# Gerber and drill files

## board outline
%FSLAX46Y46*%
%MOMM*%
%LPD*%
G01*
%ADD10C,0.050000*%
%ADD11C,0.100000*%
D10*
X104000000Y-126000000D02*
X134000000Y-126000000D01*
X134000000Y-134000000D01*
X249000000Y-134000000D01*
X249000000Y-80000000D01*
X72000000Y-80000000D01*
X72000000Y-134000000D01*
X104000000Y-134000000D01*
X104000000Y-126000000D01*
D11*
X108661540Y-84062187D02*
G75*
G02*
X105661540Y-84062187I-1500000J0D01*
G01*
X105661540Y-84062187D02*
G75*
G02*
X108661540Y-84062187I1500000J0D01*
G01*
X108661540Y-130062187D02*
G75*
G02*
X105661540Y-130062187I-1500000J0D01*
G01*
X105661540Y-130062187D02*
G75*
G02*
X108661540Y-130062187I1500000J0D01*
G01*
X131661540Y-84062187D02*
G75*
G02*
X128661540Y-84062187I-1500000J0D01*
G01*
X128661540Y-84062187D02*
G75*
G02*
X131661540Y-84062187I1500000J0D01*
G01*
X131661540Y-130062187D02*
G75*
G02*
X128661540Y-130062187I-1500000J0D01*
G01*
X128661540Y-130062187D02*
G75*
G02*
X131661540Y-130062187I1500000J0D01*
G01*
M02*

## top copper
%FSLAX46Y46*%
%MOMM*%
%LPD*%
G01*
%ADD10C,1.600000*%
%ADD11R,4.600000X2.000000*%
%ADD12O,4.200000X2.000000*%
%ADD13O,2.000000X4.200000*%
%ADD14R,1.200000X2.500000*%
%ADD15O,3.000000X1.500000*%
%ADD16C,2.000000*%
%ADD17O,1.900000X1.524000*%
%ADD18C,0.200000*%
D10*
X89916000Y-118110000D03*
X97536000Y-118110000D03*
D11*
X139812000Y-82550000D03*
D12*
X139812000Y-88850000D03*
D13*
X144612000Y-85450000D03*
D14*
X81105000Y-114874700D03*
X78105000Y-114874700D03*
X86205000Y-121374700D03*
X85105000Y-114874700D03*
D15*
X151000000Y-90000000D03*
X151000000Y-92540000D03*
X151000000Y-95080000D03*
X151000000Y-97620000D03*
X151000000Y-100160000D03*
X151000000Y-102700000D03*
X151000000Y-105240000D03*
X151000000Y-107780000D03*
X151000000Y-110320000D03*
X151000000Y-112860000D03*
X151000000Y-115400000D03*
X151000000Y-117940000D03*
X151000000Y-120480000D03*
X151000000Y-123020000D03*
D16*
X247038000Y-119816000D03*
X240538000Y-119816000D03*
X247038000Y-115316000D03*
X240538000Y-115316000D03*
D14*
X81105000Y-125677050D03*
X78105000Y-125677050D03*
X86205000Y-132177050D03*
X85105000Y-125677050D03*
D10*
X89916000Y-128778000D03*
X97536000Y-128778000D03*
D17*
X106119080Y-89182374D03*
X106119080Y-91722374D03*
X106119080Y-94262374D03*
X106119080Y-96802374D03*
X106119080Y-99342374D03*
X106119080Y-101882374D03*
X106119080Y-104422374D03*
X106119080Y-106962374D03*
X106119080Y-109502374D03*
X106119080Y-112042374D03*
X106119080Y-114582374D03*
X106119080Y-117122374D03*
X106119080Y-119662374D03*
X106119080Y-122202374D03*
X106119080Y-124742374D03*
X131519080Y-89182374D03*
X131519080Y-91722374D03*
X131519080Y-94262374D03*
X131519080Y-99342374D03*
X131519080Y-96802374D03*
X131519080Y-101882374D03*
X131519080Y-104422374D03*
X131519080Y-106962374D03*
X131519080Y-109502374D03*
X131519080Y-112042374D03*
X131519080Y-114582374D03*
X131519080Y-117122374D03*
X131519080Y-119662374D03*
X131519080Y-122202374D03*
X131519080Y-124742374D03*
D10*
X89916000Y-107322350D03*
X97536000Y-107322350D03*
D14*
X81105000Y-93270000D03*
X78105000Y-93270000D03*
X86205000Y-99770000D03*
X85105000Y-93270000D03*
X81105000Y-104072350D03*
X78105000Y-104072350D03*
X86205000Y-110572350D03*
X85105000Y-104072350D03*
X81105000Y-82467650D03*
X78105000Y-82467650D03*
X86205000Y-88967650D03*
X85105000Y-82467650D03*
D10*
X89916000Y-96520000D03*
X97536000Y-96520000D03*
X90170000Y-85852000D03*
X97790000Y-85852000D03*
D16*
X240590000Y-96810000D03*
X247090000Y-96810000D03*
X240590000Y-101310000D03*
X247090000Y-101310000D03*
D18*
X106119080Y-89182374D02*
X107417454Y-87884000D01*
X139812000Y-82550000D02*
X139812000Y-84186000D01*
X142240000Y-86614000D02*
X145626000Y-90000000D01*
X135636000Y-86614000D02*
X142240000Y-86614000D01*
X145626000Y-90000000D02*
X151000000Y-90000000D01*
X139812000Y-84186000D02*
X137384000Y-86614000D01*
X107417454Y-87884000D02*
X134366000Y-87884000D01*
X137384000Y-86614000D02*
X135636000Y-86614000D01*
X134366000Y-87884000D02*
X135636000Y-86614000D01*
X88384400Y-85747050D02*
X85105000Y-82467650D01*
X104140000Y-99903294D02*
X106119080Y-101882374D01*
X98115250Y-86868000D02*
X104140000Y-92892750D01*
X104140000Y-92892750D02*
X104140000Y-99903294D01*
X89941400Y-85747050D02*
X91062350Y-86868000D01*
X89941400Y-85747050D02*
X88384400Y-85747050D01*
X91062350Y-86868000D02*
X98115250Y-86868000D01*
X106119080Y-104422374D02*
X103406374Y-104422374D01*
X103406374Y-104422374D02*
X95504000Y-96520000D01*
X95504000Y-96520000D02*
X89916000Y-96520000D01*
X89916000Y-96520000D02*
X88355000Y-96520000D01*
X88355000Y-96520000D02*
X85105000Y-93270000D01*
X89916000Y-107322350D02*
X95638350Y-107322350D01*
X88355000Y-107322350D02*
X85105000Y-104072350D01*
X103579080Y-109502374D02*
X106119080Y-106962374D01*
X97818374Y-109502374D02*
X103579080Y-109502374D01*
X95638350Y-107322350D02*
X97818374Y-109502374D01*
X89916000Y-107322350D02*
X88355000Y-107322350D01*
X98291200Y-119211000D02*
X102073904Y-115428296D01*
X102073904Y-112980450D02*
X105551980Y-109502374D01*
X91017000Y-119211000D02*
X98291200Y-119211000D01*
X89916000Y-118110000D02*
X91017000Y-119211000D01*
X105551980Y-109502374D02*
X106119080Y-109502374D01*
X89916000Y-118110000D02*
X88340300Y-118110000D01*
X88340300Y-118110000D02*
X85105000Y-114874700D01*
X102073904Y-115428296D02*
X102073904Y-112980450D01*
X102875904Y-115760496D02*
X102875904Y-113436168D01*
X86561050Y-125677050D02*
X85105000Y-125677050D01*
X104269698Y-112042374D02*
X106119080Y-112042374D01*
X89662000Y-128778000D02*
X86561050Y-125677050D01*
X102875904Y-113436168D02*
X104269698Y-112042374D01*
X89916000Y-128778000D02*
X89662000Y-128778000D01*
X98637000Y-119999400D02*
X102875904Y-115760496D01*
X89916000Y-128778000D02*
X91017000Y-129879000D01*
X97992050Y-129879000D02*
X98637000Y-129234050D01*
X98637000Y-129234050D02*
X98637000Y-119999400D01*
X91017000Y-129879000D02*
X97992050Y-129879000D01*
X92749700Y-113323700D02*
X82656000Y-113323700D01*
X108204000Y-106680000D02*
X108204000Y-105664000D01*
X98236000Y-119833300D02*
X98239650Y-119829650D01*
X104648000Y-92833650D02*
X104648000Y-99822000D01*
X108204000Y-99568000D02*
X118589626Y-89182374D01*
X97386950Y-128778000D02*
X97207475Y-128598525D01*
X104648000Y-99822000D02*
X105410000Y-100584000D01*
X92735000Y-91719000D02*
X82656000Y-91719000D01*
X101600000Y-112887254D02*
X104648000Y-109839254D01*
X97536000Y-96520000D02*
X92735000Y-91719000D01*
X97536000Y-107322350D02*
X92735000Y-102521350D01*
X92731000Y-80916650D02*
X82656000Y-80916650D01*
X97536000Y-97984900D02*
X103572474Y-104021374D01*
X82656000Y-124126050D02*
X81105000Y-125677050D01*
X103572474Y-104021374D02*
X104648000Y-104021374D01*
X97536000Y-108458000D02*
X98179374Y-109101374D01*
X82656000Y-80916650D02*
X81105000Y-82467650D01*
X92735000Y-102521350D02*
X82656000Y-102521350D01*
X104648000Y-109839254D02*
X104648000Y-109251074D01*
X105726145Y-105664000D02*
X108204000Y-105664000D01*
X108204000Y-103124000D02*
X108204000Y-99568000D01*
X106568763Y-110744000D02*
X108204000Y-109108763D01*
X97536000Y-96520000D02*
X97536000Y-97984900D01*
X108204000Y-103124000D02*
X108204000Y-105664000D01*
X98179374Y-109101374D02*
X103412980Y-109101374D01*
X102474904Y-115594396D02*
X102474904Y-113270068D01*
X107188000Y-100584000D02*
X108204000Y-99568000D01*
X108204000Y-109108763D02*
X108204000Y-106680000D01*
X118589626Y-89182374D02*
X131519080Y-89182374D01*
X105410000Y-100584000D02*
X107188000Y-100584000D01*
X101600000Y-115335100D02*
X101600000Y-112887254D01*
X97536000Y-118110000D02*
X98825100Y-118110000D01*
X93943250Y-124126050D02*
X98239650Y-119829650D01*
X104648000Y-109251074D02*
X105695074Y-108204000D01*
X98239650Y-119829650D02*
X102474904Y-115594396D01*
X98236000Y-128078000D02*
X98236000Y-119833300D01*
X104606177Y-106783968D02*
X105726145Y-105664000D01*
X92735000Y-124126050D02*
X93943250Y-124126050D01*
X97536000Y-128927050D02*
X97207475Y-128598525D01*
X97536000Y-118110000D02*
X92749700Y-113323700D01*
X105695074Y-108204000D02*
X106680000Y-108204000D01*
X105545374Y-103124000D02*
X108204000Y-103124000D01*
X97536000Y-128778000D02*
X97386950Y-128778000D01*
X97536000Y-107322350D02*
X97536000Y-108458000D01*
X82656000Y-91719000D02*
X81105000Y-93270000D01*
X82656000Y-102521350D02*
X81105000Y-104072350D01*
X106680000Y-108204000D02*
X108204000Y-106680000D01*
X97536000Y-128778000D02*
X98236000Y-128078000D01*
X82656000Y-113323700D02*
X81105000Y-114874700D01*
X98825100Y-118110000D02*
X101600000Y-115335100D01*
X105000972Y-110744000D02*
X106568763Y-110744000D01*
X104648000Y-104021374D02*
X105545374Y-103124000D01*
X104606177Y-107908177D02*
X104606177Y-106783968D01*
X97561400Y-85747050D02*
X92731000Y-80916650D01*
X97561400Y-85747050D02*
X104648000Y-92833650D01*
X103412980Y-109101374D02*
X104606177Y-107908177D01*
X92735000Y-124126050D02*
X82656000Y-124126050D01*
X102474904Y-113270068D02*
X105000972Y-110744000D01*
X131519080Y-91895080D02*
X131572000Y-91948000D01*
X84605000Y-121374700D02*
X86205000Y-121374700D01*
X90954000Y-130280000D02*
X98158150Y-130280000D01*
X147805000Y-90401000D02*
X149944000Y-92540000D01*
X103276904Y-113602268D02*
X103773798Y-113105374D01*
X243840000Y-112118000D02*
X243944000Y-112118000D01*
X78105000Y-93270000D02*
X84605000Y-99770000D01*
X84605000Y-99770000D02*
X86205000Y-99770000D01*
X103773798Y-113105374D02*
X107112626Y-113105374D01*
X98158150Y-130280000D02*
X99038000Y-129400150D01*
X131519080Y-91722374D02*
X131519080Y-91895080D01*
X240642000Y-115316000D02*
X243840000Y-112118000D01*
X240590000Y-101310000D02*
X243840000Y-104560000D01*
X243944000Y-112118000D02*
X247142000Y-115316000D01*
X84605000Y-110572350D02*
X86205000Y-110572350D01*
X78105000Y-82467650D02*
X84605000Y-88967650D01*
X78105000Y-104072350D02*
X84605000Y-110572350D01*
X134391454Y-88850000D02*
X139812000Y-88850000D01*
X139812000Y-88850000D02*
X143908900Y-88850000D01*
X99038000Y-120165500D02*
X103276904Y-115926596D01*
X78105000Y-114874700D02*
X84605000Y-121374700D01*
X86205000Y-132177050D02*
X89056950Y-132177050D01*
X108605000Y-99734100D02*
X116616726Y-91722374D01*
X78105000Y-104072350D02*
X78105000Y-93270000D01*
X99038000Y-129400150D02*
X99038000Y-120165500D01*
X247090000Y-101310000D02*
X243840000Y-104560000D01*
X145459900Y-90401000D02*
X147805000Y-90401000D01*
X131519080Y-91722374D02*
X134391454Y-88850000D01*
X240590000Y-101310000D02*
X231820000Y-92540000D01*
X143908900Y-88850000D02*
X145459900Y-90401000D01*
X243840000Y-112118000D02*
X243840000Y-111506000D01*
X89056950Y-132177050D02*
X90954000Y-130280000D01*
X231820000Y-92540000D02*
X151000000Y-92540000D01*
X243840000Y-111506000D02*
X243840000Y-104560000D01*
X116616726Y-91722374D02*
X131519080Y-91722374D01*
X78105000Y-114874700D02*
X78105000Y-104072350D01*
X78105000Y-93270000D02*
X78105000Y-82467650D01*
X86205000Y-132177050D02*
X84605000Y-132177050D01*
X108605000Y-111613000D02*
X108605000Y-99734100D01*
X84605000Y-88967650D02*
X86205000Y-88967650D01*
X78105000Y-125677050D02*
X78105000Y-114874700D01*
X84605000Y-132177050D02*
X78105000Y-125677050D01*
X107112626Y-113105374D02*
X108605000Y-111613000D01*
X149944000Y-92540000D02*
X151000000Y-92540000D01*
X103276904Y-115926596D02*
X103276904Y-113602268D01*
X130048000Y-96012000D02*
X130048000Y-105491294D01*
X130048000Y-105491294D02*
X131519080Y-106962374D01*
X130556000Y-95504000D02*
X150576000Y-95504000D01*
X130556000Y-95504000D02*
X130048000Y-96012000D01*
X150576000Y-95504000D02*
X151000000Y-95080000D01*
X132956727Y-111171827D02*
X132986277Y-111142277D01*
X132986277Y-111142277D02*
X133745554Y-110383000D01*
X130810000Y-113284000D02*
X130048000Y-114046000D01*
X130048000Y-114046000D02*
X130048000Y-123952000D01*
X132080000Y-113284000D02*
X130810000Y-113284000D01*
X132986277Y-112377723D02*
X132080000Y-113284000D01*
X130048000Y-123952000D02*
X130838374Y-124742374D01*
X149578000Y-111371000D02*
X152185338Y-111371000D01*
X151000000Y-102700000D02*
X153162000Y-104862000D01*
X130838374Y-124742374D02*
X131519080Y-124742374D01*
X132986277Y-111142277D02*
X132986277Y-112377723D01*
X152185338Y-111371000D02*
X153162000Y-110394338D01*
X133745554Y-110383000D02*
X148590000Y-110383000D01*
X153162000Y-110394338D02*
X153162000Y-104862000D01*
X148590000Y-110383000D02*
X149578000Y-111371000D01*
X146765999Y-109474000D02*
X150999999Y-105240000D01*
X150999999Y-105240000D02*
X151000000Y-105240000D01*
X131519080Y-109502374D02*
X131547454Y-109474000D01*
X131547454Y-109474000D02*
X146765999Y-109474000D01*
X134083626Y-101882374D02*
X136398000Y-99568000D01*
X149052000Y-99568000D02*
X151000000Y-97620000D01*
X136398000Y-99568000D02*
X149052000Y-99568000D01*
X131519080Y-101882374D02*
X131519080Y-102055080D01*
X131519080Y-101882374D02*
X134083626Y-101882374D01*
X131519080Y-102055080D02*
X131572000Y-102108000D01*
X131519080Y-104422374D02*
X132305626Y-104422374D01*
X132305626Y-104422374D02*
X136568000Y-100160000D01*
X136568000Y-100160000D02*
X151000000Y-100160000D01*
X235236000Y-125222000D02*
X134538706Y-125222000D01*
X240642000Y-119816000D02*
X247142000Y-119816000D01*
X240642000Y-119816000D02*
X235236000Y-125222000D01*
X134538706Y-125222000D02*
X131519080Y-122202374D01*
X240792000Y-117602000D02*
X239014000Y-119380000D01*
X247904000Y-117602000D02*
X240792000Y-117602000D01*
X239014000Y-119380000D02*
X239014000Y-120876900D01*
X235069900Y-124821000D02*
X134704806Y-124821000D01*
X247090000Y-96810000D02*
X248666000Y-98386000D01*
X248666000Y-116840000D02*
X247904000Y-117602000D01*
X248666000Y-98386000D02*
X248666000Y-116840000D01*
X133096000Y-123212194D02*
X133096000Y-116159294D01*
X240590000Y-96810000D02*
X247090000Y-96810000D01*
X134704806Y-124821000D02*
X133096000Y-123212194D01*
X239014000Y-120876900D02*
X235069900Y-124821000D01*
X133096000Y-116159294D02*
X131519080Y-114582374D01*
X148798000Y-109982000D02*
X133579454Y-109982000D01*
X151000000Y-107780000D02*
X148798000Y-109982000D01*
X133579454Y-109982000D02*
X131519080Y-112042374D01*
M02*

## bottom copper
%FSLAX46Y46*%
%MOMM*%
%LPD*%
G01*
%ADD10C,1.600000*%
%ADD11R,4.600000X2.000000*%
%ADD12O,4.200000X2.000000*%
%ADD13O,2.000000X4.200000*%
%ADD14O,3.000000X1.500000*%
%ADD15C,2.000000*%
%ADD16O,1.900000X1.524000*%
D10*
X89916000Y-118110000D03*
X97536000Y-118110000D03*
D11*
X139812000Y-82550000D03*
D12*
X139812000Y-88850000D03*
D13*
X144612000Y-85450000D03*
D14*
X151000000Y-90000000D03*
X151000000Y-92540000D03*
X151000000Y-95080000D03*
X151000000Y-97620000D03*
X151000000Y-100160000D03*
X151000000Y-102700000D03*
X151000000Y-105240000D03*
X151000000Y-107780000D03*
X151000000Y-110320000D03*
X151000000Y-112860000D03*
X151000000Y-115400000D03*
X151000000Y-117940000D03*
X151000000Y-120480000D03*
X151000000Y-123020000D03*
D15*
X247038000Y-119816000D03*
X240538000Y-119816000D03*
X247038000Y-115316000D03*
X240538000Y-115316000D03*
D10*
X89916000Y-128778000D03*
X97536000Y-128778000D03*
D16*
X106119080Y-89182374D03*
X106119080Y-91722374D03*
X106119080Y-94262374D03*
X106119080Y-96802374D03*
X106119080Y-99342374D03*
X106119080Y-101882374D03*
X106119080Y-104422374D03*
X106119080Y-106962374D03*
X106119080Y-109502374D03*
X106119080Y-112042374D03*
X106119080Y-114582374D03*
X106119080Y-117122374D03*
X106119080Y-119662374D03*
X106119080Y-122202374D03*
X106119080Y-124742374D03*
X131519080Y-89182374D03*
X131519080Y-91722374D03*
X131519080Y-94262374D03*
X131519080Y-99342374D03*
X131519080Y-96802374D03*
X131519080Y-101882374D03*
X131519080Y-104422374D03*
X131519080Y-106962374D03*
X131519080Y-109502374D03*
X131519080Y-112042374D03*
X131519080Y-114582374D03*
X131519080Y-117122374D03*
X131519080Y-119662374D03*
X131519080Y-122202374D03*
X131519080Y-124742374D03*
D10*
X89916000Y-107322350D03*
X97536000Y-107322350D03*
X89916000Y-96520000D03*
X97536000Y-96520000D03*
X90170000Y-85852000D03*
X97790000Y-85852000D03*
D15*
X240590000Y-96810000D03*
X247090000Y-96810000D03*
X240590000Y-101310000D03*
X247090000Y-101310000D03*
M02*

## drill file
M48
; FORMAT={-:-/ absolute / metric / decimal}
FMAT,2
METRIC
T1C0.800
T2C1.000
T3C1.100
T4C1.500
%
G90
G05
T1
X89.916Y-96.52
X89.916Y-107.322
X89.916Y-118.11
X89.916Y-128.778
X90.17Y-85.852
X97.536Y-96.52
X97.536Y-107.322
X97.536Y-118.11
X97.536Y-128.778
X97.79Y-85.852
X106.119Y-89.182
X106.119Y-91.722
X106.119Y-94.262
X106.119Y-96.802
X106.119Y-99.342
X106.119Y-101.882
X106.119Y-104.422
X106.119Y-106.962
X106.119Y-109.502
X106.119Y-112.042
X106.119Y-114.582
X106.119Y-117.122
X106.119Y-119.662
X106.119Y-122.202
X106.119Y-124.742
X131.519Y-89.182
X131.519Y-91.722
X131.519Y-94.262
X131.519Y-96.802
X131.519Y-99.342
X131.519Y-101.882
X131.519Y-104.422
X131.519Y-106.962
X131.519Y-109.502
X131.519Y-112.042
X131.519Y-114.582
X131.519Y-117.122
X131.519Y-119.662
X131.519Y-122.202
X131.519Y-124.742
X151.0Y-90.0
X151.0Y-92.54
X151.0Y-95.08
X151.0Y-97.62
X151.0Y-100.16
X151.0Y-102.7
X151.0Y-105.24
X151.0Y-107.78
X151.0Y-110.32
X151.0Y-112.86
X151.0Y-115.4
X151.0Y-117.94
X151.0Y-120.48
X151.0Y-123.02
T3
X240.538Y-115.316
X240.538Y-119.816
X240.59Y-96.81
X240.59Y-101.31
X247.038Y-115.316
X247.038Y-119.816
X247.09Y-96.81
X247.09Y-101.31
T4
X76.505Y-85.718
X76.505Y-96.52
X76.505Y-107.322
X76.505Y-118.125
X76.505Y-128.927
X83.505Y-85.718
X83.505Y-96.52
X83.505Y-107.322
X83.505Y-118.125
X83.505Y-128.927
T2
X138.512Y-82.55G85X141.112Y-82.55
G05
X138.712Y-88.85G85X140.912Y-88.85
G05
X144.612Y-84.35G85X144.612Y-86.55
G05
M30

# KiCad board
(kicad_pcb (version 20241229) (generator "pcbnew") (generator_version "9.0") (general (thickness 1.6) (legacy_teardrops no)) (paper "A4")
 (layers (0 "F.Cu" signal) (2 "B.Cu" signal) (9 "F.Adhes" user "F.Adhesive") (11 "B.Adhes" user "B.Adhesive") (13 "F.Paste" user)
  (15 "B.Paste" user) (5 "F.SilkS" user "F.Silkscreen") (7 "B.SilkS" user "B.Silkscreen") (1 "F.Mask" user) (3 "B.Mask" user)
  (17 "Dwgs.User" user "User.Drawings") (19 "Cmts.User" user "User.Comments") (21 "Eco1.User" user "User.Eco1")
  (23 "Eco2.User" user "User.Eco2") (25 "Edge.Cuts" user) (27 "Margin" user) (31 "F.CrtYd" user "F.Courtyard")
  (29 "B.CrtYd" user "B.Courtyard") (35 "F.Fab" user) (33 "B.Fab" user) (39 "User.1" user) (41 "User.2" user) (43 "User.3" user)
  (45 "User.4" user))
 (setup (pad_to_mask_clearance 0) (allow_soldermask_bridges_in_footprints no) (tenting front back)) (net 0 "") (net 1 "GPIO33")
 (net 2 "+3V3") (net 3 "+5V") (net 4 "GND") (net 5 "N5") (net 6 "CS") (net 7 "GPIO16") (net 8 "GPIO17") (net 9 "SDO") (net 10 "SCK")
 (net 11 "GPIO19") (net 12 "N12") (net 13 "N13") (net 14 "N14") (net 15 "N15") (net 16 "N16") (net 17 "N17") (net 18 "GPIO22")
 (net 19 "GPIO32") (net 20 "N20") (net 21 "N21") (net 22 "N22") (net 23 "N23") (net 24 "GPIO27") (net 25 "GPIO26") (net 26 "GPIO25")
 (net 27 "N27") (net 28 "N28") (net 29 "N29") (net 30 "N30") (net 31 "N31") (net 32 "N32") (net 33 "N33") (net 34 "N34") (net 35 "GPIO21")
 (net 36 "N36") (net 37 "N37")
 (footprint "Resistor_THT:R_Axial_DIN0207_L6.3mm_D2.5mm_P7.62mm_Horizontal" (layer "F.Cu") (at 89.916 118.11)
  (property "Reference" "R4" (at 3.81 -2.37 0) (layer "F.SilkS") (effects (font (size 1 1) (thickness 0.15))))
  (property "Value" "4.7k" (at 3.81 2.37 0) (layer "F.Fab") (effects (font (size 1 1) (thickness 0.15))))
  (pad "1" thru_hole circle (at 0 0) (size 1.6 1.6) (drill 0.8) (layers "*.Cu" "*.Mask") (remove_unused_layers no) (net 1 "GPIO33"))
  (pad "2" thru_hole circle (at 7.62 0) (size 1.6 1.6) (drill 0.8) (layers "*.Cu" "*.Mask") (remove_unused_layers no) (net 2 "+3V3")))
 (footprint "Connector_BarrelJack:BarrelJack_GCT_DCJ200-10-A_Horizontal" (layer "F.Cu") (at 139.812 82.55)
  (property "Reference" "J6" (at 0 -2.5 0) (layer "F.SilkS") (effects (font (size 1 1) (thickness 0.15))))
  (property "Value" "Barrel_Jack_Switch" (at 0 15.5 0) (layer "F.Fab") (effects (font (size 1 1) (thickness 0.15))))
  (pad "1" thru_hole rect (at 0 0) (size 4.6 2) (drill oval 3.6 1) (layers "*.Cu" "*.Mask") (remove_unused_layers no) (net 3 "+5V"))
  (pad "2" thru_hole oval (at 0 6.3) (size 4.2 2) (drill oval 3.2 1) (layers "*.Cu" "*.Mask") (remove_unused_layers no) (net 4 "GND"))
  (pad "3" thru_hole oval (at 4.8 2.9) (size 2 4.2) (drill oval 1 3.2) (layers "*.Cu" "*.Mask") (remove_unused_layers no) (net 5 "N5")))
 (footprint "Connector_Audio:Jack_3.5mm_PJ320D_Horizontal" (layer "F.Cu") (at 81.28 118.1247)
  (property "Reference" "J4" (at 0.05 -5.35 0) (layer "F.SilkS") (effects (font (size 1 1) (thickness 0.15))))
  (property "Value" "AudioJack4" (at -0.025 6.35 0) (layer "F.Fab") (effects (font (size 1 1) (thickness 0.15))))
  (pad "" np_thru_hole circle (at -4.775 0) (size 1.5 1.5) (drill 1.5) (layers "*.Cu" "*.Mask"))
  (pad "" np_thru_hole circle (at 2.225 0) (size 1.5 1.5) (drill 1.5) (layers "*.Cu" "*.Mask"))
  (pad "R1" smd rect (at -0.175 -3.25) (size 1.2 2.5) (layers "F.Cu" "F.Mask" "F.Paste") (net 2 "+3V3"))
  (pad "R2" smd rect (at -3.175 -3.25) (size 1.2 2.5) (layers "F.Cu" "F.Mask" "F.Paste") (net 4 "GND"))
  (pad "S" smd rect (at 4.925 3.25) (size 1.2 2.5) (layers "F.Cu" "F.Mask" "F.Paste") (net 4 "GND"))
  (pad "T" smd rect (at 3.825 -3.25) (size 1.2 2.5) (layers "F.Cu" "F.Mask" "F.Paste") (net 1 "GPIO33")))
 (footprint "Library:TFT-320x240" (layer "F.Cu") (at 151 106.51 -90)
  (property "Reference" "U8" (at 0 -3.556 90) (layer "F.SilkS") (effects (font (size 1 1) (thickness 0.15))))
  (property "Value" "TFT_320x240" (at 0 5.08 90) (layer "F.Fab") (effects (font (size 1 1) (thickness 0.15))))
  (pad "1" thru_hole oval (at -16.51 0 270) (size 1.5 3) (drill 0.8) (layers "*.Cu" "*.Mask") (remove_unused_layers no) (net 3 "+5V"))
  (pad "2" thru_hole oval (at -13.97 0 270) (size 1.5 3) (drill 0.8) (layers "*.Cu" "*.Mask") (remove_unused_layers no) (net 4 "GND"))
  (pad "3" thru_hole oval (at -11.43 0 270) (size 1.5 3) (drill 0.8) (layers "*.Cu" "*.Mask") (remove_unused_layers no) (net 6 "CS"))
  (pad "4" thru_hole oval (at -8.89 0 270) (size 1.5 3) (drill 0.8) (layers "*.Cu" "*.Mask") (remove_unused_layers no) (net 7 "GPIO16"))
  (pad "5" thru_hole oval (at -6.35 0 270) (size 1.5 3) (drill 0.8) (layers "*.Cu" "*.Mask") (remove_unused_layers no) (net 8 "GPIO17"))
  (pad "6" thru_hole oval (at -3.81 0 270) (size 1.5 3) (drill 0.8) (layers "*.Cu" "*.Mask") (remove_unused_layers no) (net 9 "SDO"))
  (pad "7" thru_hole oval (at -1.27 0 270) (size 1.5 3) (drill 0.8) (layers "*.Cu" "*.Mask") (remove_unused_layers no) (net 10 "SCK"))
  (pad "8" thru_hole oval (at 1.27 0 270) (size 1.5 3) (drill 0.8) (layers "*.Cu" "*.Mask") (remove_unused_layers no) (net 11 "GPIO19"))
  (pad "9" thru_hole oval (at 3.81 0 270) (size 1.5 3) (drill 0.8) (layers "*.Cu" "*.Mask") (remove_unused_layers no) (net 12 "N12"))
  (pad "10" thru_hole oval (at 6.35 0 270) (size 1.5 3) (drill 0.8) (layers "*.Cu" "*.Mask") (remove_unused_layers no) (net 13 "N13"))
  (pad "11" thru_hole oval (at 8.89 0 270) (size 1.5 3) (drill 0.8) (layers "*.Cu" "*.Mask") (remove_unused_layers no) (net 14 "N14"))
  (pad "12" thru_hole oval (at 11.43 0 270) (size 1.5 3) (drill 0.8) (layers "*.Cu" "*.Mask") (remove_unused_layers no) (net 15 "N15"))
  (pad "13" thru_hole oval (at 13.97 0 270) (size 1.5 3) (drill 0.8) (layers "*.Cu" "*.Mask") (remove_unused_layers no) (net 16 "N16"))
  (pad "14" thru_hole oval (at 16.51 0 270) (size 1.5 3) (drill 0.8) (layers "*.Cu" "*.Mask") (remove_unused_layers no) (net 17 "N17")))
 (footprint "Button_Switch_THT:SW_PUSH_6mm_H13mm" (layer "F.Cu") (at 247.038 119.816 180)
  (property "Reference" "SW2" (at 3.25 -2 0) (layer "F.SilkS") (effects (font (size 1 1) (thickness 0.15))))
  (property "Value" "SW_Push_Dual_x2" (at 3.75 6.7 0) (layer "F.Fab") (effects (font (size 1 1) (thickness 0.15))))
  (pad "1" thru_hole circle (at 0 0 270) (size 2 2) (drill 1.1) (layers "*.Cu" "*.Mask") (remove_unused_layers no) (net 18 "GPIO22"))
  (pad "1" thru_hole circle (at 6.5 0 270) (size 2 2) (drill 1.1) (layers "*.Cu" "*.Mask") (remove_unused_layers no) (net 18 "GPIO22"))
  (pad "2" thru_hole circle (at 0 4.5 270) (size 2 2) (drill 1.1) (layers "*.Cu" "*.Mask") (remove_unused_layers no) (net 4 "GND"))
  (pad "2" thru_hole circle (at 6.5 4.5 270) (size 2 2) (drill 1.1) (layers "*.Cu" "*.Mask") (remove_unused_layers no) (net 4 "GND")))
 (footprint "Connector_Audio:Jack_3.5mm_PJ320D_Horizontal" (layer "F.Cu") (at 81.28 128.92705)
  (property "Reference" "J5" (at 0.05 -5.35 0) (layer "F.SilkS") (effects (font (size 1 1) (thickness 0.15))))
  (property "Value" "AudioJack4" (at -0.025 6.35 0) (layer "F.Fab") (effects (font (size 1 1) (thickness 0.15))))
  (pad "" np_thru_hole circle (at -4.775 0) (size 1.5 1.5) (drill 1.5) (layers "*.Cu" "*.Mask"))
  (pad "" np_thru_hole circle (at 2.225 0) (size 1.5 1.5) (drill 1.5) (layers "*.Cu" "*.Mask"))
  (pad "R1" smd rect (at -0.175 -3.25) (size 1.2 2.5) (layers "F.Cu" "F.Mask" "F.Paste") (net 2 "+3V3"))
  (pad "R2" smd rect (at -3.175 -3.25) (size 1.2 2.5) (layers "F.Cu" "F.Mask" "F.Paste") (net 4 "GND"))
  (pad "S" smd rect (at 4.925 3.25) (size 1.2 2.5) (layers "F.Cu" "F.Mask" "F.Paste") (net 4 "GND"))
  (pad "T" smd rect (at 3.825 -3.25) (size 1.2 2.5) (layers "F.Cu" "F.Mask" "F.Paste") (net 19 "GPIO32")))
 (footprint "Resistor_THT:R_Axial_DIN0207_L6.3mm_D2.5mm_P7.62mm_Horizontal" (layer "F.Cu") (at 89.916 128.778)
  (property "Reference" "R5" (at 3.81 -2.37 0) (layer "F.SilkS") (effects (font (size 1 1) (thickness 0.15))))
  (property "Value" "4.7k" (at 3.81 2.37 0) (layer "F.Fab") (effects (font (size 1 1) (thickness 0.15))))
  (pad "1" thru_hole circle (at 0 0) (size 1.6 1.6) (drill 0.8) (layers "*.Cu" "*.Mask") (remove_unused_layers no) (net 19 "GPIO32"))
  (pad "2" thru_hole circle (at 7.62 0) (size 1.6 1.6) (drill 0.8) (layers "*.Cu" "*.Mask") (remove_unused_layers no) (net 2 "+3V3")))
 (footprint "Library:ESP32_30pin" (layer "F.Cu") (at 118.59154 107.202187 90)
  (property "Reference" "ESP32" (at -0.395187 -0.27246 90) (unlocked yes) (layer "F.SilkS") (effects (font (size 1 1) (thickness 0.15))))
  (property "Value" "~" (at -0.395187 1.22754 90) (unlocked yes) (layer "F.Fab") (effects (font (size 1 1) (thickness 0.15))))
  (fp_circle (center 23.14 -11.43) (end 24.64 -11.43) (stroke (width 0.1) (type default)) (fill no) (layer "Edge.Cuts"))
  (fp_circle (center -22.86 -11.43) (end -21.36 -11.43) (stroke (width 0.1) (type default)) (fill no) (layer "Edge.Cuts"))
  (fp_circle (center 23.14 11.57) (end 24.64 11.57) (stroke (width 0.1) (type default)) (fill no) (layer "Edge.Cuts"))
  (fp_circle (center -22.86 11.57) (end -21.36 11.57) (stroke (width 0.1) (type default)) (fill no) (layer "Edge.Cuts"))
  (pad "1" thru_hole oval (at 18.019813 -12.47246 90) (size 1.524 1.9) (drill 0.8) (layers "*.Cu" "*.Mask") (remove_unused_layers no)
   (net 3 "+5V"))
  (pad "2" thru_hole oval (at 15.479813 -12.47246 90) (size 1.524 1.9) (drill 0.8) (layers "*.Cu" "*.Mask") (remove_unused_layers no)
   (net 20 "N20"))
  (pad "3" thru_hole oval (at 12.939813 -12.47246 90) (size 1.524 1.9) (drill 0.8) (layers "*.Cu" "*.Mask") (remove_unused_layers no)
   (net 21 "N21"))
  (pad "4" thru_hole oval (at 10.399813 -12.47246 90) (size 1.524 1.9) (drill 0.8) (layers "*.Cu" "*.Mask") (remove_unused_layers no)
   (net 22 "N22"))
  (pad "5" thru_hole oval (at 7.859813 -12.47246 90) (size 1.524 1.9) (drill 0.8) (layers "*.Cu" "*.Mask") (remove_unused_layers no)
   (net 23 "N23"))
  (pad "6" thru_hole oval (at 5.319813 -12.47246 90) (size 1.524 1.9) (drill 0.8) (layers "*.Cu" "*.Mask") (remove_unused_layers no)
   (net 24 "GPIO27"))
  (pad "7" thru_hole oval (at 2.779813 -12.47246 90) (size 1.524 1.9) (drill 0.8) (layers "*.Cu" "*.Mask") (remove_unused_layers no)
   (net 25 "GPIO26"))
  (pad "8" thru_hole oval (at 0.239813 -12.47246 90) (size 1.524 1.9) (drill 0.8) (layers "*.Cu" "*.Mask") (remove_unused_layers no)
   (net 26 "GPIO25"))
  (pad "9" thru_hole oval (at -2.300187 -12.47246 90) (size 1.524 1.9) (drill 0.8) (layers "*.Cu" "*.Mask") (remove_unused_layers no)
   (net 1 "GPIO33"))
  (pad "10" thru_hole oval (at -4.840187 -12.47246 90) (size 1.524 1.9) (drill 0.8) (layers "*.Cu" "*.Mask") (remove_unused_layers no)
   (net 19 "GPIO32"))
  (pad "11" thru_hole oval (at -7.380187 -12.47246 90) (size 1.524 1.9) (drill 0.8) (layers "*.Cu" "*.Mask") (remove_unused_layers no)
   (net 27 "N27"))
  (pad "12" thru_hole oval (at -9.920187 -12.47246 90) (size 1.524 1.9) (drill 0.8) (layers "*.Cu" "*.Mask") (remove_unused_layers no)
   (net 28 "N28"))
  (pad "13" thru_hole oval (at -12.460187 -12.47246 90) (size 1.524 1.9) (drill 0.8) (layers "*.Cu" "*.Mask") (remove_unused_layers no)
   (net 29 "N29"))
  (pad "14" thru_hole oval (at -15.000187 -12.47246 90) (size 1.524 1.9) (drill 0.8) (layers "*.Cu" "*.Mask") (remove_unused_layers no)
   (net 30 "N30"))
  (pad "15" thru_hole oval (at -17.540187 -12.47246 90) (size 1.524 1.9) (drill 0.8) (layers "*.Cu" "*.Mask") (remove_unused_layers no)
   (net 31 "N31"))
  (pad "16" thru_hole oval (at 18.019813 12.92754 90) (size 1.524 1.9) (drill 0.8) (layers "*.Cu" "*.Mask") (remove_unused_layers no)
   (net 2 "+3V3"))
  (pad "17" thru_hole oval (at 15.479813 12.92754 90) (size 1.524 1.9) (drill 0.8) (layers "*.Cu" "*.Mask") (remove_unused_layers no)
   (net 4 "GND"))
  (pad "18" thru_hole oval (at 12.939813 12.92754 90) (size 1.524 1.9) (drill 0.8) (layers "*.Cu" "*.Mask") (remove_unused_layers no)
   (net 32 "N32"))
  (pad "19" thru_hole oval (at 7.859813 12.92754 90) (size 1.524 1.9) (drill 0.8) (layers "*.Cu" "*.Mask") (remove_unused_layers no)
   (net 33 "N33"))
  (pad "20" thru_hole oval (at 10.399813 12.92754 90) (size 1.524 1.9) (drill 0.8) (layers "*.Cu" "*.Mask") (remove_unused_layers no)
   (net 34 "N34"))
  (pad "21" thru_hole oval (at 5.319813 12.92754 90) (size 1.524 1.9) (drill 0.8) (layers "*.Cu" "*.Mask") (remove_unused_layers no)
   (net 7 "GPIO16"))
  (pad "22" thru_hole oval (at 2.779813 12.92754 90) (size 1.524 1.9) (drill 0.8) (layers "*.Cu" "*.Mask") (remove_unused_layers no)
   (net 8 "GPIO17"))
  (pad "23" thru_hole oval (at 0.239813 12.92754 90) (size 1.524 1.9) (drill 0.8) (layers "*.Cu" "*.Mask") (remove_unused_layers no)
   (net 6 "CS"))
  (pad "24" thru_hole oval (at -2.300187 12.92754 90) (size 1.524 1.9) (drill 0.8) (layers "*.Cu" "*.Mask") (remove_unused_layers no)
   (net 10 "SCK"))
  (pad "25" thru_hole oval (at -4.840187 12.92754 90) (size 1.524 1.9) (drill 0.8) (layers "*.Cu" "*.Mask") (remove_unused_layers no)
   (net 11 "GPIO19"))
  (pad "26" thru_hole oval (at -7.380187 12.92754 90) (size 1.524 1.9) (drill 0.8) (layers "*.Cu" "*.Mask") (remove_unused_layers no)
   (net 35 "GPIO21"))
  (pad "27" thru_hole oval (at -9.920187 12.92754 90) (size 1.524 1.9) (drill 0.8) (layers "*.Cu" "*.Mask") (remove_unused_layers no)
   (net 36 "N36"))
  (pad "28" thru_hole oval (at -12.460187 12.92754 90) (size 1.524 1.9) (drill 0.8) (layers "*.Cu" "*.Mask") (remove_unused_layers no)
   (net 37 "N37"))
  (pad "29" thru_hole oval (at -15.000187 12.92754 90) (size 1.524 1.9) (drill 0.8) (layers "*.Cu" "*.Mask") (remove_unused_layers no)
   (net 18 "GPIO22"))
  (pad "30" thru_hole oval (at -17.540187 12.92754 90) (size 1.524 1.9) (drill 0.8) (layers "*.Cu" "*.Mask") (remove_unused_layers no)
   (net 9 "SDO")))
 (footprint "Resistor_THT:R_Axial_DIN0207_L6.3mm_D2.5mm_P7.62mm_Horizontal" (layer "F.Cu") (at 89.916 107.32235)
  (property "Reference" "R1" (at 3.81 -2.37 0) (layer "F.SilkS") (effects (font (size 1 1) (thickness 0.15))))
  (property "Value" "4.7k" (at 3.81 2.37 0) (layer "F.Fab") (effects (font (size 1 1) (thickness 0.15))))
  (pad "1" thru_hole circle (at 0 0) (size 1.6 1.6) (drill 0.8) (layers "*.Cu" "*.Mask") (remove_unused_layers no) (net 26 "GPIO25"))
  (pad "2" thru_hole circle (at 7.62 0) (size 1.6 1.6) (drill 0.8) (layers "*.Cu" "*.Mask") (remove_unused_layers no) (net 2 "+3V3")))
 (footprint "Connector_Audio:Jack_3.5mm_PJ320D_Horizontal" (layer "F.Cu") (at 81.28 96.52)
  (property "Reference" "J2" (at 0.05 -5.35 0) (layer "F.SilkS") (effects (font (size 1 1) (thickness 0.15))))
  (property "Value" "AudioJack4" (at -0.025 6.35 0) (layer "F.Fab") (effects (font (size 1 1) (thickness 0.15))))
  (pad "" np_thru_hole circle (at -4.775 0) (size 1.5 1.5) (drill 1.5) (layers "*.Cu" "*.Mask"))
  (pad "" np_thru_hole circle (at 2.225 0) (size 1.5 1.5) (drill 1.5) (layers "*.Cu" "*.Mask"))
  (pad "R1" smd rect (at -0.175 -3.25) (size 1.2 2.5) (layers "F.Cu" "F.Mask" "F.Paste") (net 2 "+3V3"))
  (pad "R2" smd rect (at -3.175 -3.25) (size 1.2 2.5) (layers "F.Cu" "F.Mask" "F.Paste") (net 4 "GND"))
  (pad "S" smd rect (at 4.925 3.25) (size 1.2 2.5) (layers "F.Cu" "F.Mask" "F.Paste") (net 4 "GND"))
  (pad "T" smd rect (at 3.825 -3.25) (size 1.2 2.5) (layers "F.Cu" "F.Mask" "F.Paste") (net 25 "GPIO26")))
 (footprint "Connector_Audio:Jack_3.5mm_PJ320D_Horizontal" (layer "F.Cu") (at 81.28 107.32235)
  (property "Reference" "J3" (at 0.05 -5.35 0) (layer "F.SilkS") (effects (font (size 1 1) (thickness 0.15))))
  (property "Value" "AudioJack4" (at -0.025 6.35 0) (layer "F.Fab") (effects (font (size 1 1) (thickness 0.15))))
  (pad "" np_thru_hole circle (at -4.775 0) (size 1.5 1.5) (drill 1.5) (layers "*.Cu" "*.Mask"))
  (pad "" np_thru_hole circle (at 2.225 0) (size 1.5 1.5) (drill 1.5) (layers "*.Cu" "*.Mask"))
  (pad "R1" smd rect (at -0.175 -3.25) (size 1.2 2.5) (layers "F.Cu" "F.Mask" "F.Paste") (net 2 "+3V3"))
  (pad "R2" smd rect (at -3.175 -3.25) (size 1.2 2.5) (layers "F.Cu" "F.Mask" "F.Paste") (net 4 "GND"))
  (pad "S" smd rect (at 4.925 3.25) (size 1.2 2.5) (layers "F.Cu" "F.Mask" "F.Paste") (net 4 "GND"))
  (pad "T" smd rect (at 3.825 -3.25) (size 1.2 2.5) (layers "F.Cu" "F.Mask" "F.Paste") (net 26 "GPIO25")))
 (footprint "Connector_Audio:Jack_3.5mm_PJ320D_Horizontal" (layer "F.Cu") (at 81.28 85.71765)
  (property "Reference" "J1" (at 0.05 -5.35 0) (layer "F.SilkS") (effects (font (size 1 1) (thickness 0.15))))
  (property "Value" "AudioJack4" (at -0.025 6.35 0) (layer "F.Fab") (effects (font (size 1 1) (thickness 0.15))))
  (pad "" np_thru_hole circle (at -4.775 0) (size 1.5 1.5) (drill 1.5) (layers "*.Cu" "*.Mask"))
  (pad "" np_thru_hole circle (at 2.225 0) (size 1.5 1.5) (drill 1.5) (layers "*.Cu" "*.Mask"))
  (pad "R1" smd rect (at -0.175 -3.25) (size 1.2 2.5) (layers "F.Cu" "F.Mask" "F.Paste") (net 2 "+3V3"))
  (pad "R2" smd rect (at -3.175 -3.25) (size 1.2 2.5) (layers "F.Cu" "F.Mask" "F.Paste") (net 4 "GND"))
  (pad "S" smd rect (at 4.925 3.25) (size 1.2 2.5) (layers "F.Cu" "F.Mask" "F.Paste") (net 4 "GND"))
  (pad "T" smd rect (at 3.825 -3.25) (size 1.2 2.5) (layers "F.Cu" "F.Mask" "F.Paste") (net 24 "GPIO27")))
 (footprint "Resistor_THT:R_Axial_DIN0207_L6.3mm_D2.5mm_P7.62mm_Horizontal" (layer "F.Cu") (at 89.916 96.52)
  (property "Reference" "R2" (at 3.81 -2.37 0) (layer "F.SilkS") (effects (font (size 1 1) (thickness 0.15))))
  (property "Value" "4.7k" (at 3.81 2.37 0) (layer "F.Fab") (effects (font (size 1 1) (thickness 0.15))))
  (pad "1" thru_hole circle (at 0 0) (size 1.6 1.6) (drill 0.8) (layers "*.Cu" "*.Mask") (remove_unused_layers no) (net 25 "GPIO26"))
  (pad "2" thru_hole circle (at 7.62 0) (size 1.6 1.6) (drill 0.8) (layers "*.Cu" "*.Mask") (remove_unused_layers no) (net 2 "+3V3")))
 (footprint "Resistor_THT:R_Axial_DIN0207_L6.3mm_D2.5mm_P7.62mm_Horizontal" (layer "F.Cu") (at 90.17 85.852)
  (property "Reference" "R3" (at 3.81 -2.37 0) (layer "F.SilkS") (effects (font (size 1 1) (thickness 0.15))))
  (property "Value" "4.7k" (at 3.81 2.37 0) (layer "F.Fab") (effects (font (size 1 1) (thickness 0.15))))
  (pad "1" thru_hole circle (at 0 0) (size 1.6 1.6) (drill 0.8) (layers "*.Cu" "*.Mask") (remove_unused_layers no) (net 24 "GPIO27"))
  (pad "2" thru_hole circle (at 7.62 0) (size 1.6 1.6) (drill 0.8) (layers "*.Cu" "*.Mask") (remove_unused_layers no) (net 2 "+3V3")))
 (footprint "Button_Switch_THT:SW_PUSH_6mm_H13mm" (layer "F.Cu") (at 240.59 96.81)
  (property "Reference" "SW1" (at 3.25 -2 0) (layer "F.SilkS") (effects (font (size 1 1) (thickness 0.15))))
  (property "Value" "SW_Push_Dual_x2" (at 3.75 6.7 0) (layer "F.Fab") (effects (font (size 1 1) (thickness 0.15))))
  (pad "1" thru_hole circle (at 0 0 90) (size 2 2) (drill 1.1) (layers "*.Cu" "*.Mask") (remove_unused_layers no) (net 35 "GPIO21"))
  (pad "1" thru_hole circle (at 6.5 0 90) (size 2 2) (drill 1.1) (layers "*.Cu" "*.Mask") (remove_unused_layers no) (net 35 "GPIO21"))
  (pad "2" thru_hole circle (at 0 4.5 90) (size 2 2) (drill 1.1) (layers "*.Cu" "*.Mask") (remove_unused_layers no) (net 4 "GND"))
  (pad "2" thru_hole circle (at 6.5 4.5 90) (size 2 2) (drill 1.1) (layers "*.Cu" "*.Mask") (remove_unused_layers no) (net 4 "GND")))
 (gr_poly
  (pts (xy 104 126) (xy 134 126) (xy 134 134) (xy 249 134) (xy 249 80) (xy 72 80) (xy 72 134) (xy 104 134))
  (stroke (width 0.05) (type solid)) (fill no) (layer "Edge.Cuts"))
 (segment (start 106.11908 89.182374) (end 107.417454 87.884) (width 0.2) (layer "F.Cu") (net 3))
 (segment (start 139.812 82.55) (end 139.812 84.186) (width 0.2) (layer "F.Cu") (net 3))
 (segment (start 142.24 86.614) (end 145.626 90) (width 0.2) (layer "F.Cu") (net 3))
 (segment (start 135.636 86.614) (end 142.24 86.614) (width 0.2) (layer "F.Cu") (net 3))
 (segment (start 145.626 90) (end 151 90) (width 0.2) (layer "F.Cu") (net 3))
 (segment (start 139.812 84.186) (end 137.384 86.614) (width 0.2) (layer "F.Cu") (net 3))
 (segment (start 107.417454 87.884) (end 134.366 87.884) (width 0.2) (layer "F.Cu") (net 3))
 (segment (start 137.384 86.614) (end 135.636 86.614) (width 0.2) (layer "F.Cu") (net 3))
 (segment (start 134.366 87.884) (end 135.636 86.614) (width 0.2) (layer "F.Cu") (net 3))
 (segment (start 88.3844 85.74705) (end 85.105 82.46765) (width 0.2) (layer "F.Cu") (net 24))
 (segment (start 104.14 99.903294) (end 106.11908 101.882374) (width 0.2) (layer "F.Cu") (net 24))
 (segment (start 98.11525 86.868) (end 104.14 92.89275) (width 0.2) (layer "F.Cu") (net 24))
 (segment (start 104.14 92.89275) (end 104.14 99.903294) (width 0.2) (layer "F.Cu") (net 24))
 (segment (start 89.9414 85.74705) (end 91.06235 86.868) (width 0.2) (layer "F.Cu") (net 24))
 (segment (start 89.9414 85.74705) (end 88.3844 85.74705) (width 0.2) (layer "F.Cu") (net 24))
 (segment (start 91.06235 86.868) (end 98.11525 86.868) (width 0.2) (layer "F.Cu") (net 24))
 (segment (start 106.11908 104.422374) (end 103.406374 104.422374) (width 0.2) (layer "F.Cu") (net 25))
 (segment (start 103.406374 104.422374) (end 95.504 96.52) (width 0.2) (layer "F.Cu") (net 25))
 (segment (start 95.504 96.52) (end 89.916 96.52) (width 0.2) (layer "F.Cu") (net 25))
 (segment (start 89.916 96.52) (end 88.355 96.52) (width 0.2) (layer "F.Cu") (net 25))
 (segment (start 88.355 96.52) (end 85.105 93.27) (width 0.2) (layer "F.Cu") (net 25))
 (segment (start 89.916 107.32235) (end 95.63835 107.32235) (width 0.2) (layer "F.Cu") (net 26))
 (segment (start 88.355 107.32235) (end 85.105 104.07235) (width 0.2) (layer "F.Cu") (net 26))
 (segment (start 103.57908 109.502374) (end 106.11908 106.962374) (width 0.2) (layer "F.Cu") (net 26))
 (segment (start 97.818374 109.502374) (end 103.57908 109.502374) (width 0.2) (layer "F.Cu") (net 26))
 (segment (start 95.63835 107.32235) (end 97.818374 109.502374) (width 0.2) (layer "F.Cu") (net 26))
 (segment (start 89.916 107.32235) (end 88.355 107.32235) (width 0.2) (layer "F.Cu") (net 26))
 (segment (start 98.2912 119.211) (end 102.073904 115.428296) (width 0.2) (layer "F.Cu") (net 1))
 (segment (start 102.073904 112.98045) (end 105.55198 109.502374) (width 0.2) (layer "F.Cu") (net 1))
 (segment (start 91.017 119.211) (end 98.2912 119.211) (width 0.2) (layer "F.Cu") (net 1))
 (segment (start 89.916 118.11) (end 91.017 119.211) (width 0.2) (layer "F.Cu") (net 1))
 (segment (start 105.55198 109.502374) (end 106.11908 109.502374) (width 0.2) (layer "F.Cu") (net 1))
 (segment (start 89.916 118.11) (end 88.3403 118.11) (width 0.2) (layer "F.Cu") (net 1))
 (segment (start 88.3403 118.11) (end 85.105 114.8747) (width 0.2) (layer "F.Cu") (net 1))
 (segment (start 102.073904 115.428296) (end 102.073904 112.98045) (width 0.2) (layer "F.Cu") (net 1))
 (segment (start 102.875904 115.760496) (end 102.875904 113.436168) (width 0.2) (layer "F.Cu") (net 19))
 (segment (start 86.56105 125.67705) (end 85.105 125.67705) (width 0.2) (layer "F.Cu") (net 19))
 (segment (start 104.269698 112.042374) (end 106.11908 112.042374) (width 0.2) (layer "F.Cu") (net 19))
 (segment (start 89.662 128.778) (end 86.56105 125.67705) (width 0.2) (layer "F.Cu") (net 19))
 (segment (start 102.875904 113.436168) (end 104.269698 112.042374) (width 0.2) (layer "F.Cu") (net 19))
 (segment (start 89.916 128.778) (end 89.662 128.778) (width 0.2) (layer "F.Cu") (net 19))
 (segment (start 98.637 119.9994) (end 102.875904 115.760496) (width 0.2) (layer "F.Cu") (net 19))
 (segment (start 89.916 128.778) (end 91.017 129.879) (width 0.2) (layer "F.Cu") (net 19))
 (segment (start 97.99205 129.879) (end 98.637 129.23405) (width 0.2) (layer "F.Cu") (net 19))
 (segment (start 98.637 129.23405) (end 98.637 119.9994) (width 0.2) (layer "F.Cu") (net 19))
 (segment (start 91.017 129.879) (end 97.99205 129.879) (width 0.2) (layer "F.Cu") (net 19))
 (segment (start 92.7497 113.3237) (end 82.656 113.3237) (width 0.2) (layer "F.Cu") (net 2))
 (segment (start 108.204 106.68) (end 108.204 105.664) (width 0.2) (layer "F.Cu") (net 2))
 (segment (start 98.236 119.8333) (end 98.23965 119.82965) (width 0.2) (layer "F.Cu") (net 2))
 (segment (start 104.648 92.83365) (end 104.648 99.822) (width 0.2) (layer "F.Cu") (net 2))
 (segment (start 108.204 99.568) (end 118.589626 89.182374) (width 0.2) (layer "F.Cu") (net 2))
 (segment (start 97.38695 128.778) (end 97.207475 128.598525) (width 0.2) (layer "F.Cu") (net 2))
 (segment (start 104.648 99.822) (end 105.41 100.584) (width 0.2) (layer "F.Cu") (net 2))
 (segment (start 92.735 91.719) (end 82.656 91.719) (width 0.2) (layer "F.Cu") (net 2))
 (segment (start 101.6 112.887254) (end 104.648 109.839254) (width 0.2) (layer "F.Cu") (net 2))
 (segment (start 97.536 96.52) (end 92.735 91.719) (width 0.2) (layer "F.Cu") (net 2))
 (segment (start 97.536 107.32235) (end 92.735 102.52135) (width 0.2) (layer "F.Cu") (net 2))
 (segment (start 92.731 80.91665) (end 82.656 80.91665) (width 0.2) (layer "F.Cu") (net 2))
 (segment (start 97.536 97.9849) (end 103.572474 104.021374) (width 0.2) (layer "F.Cu") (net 2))
 (segment (start 82.656 124.12605) (end 81.105 125.67705) (width 0.2) (layer "F.Cu") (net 2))
 (segment (start 103.572474 104.021374) (end 104.648 104.021374) (width 0.2) (layer "F.Cu") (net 2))
 (segment (start 97.536 108.458) (end 98.179374 109.101374) (width 0.2) (layer "F.Cu") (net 2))
 (segment (start 82.656 80.91665) (end 81.105 82.46765) (width 0.2) (layer "F.Cu") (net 2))
 (segment (start 92.735 102.52135) (end 82.656 102.52135) (width 0.2) (layer "F.Cu") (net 2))
 (segment (start 104.648 109.839254) (end 104.648 109.251074) (width 0.2) (layer "F.Cu") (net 2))
 (segment (start 105.726145 105.664) (end 108.204 105.664) (width 0.2) (layer "F.Cu") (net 2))
 (segment (start 108.204 103.124) (end 108.204 99.568) (width 0.2) (layer "F.Cu") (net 2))
 (segment (start 106.568763 110.744) (end 108.204 109.108763) (width 0.2) (layer "F.Cu") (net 2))
 (segment (start 97.536 96.52) (end 97.536 97.9849) (width 0.2) (layer "F.Cu") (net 2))
 (segment (start 108.204 103.124) (end 108.204 105.664) (width 0.2) (layer "F.Cu") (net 2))
 (segment (start 98.179374 109.101374) (end 103.41298 109.101374) (width 0.2) (layer "F.Cu") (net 2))
 (segment (start 102.474904 115.594396) (end 102.474904 113.270068) (width 0.2) (layer "F.Cu") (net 2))
 (segment (start 107.188 100.584) (end 108.204 99.568) (width 0.2) (layer "F.Cu") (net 2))
 (segment (start 108.204 109.108763) (end 108.204 106.68) (width 0.2) (layer "F.Cu") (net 2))
 (segment (start 118.589626 89.182374) (end 131.51908 89.182374) (width 0.2) (layer "F.Cu") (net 2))
 (segment (start 105.41 100.584) (end 107.188 100.584) (width 0.2) (layer "F.Cu") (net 2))
 (segment (start 101.6 115.3351) (end 101.6 112.887254) (width 0.2) (layer "F.Cu") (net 2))
 (segment (start 97.536 118.11) (end 98.8251 118.11) (width 0.2) (layer "F.Cu") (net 2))
 (segment (start 93.94325 124.12605) (end 98.23965 119.82965) (width 0.2) (layer "F.Cu") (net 2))
 (segment (start 104.648 109.251074) (end 105.695074 108.204) (width 0.2) (layer "F.Cu") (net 2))
 (segment (start 98.23965 119.82965) (end 102.474904 115.594396) (width 0.2) (layer "F.Cu") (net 2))
 (segment (start 98.236 128.078) (end 98.236 119.8333) (width 0.2) (layer "F.Cu") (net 2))
 (segment (start 104.606177 106.783968) (end 105.726145 105.664) (width 0.2) (layer "F.Cu") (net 2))
 (segment (start 92.735 124.12605) (end 93.94325 124.12605) (width 0.2) (layer "F.Cu") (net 2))
 (segment (start 97.536 128.92705) (end 97.207475 128.598525) (width 0.2) (layer "F.Cu") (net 2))
 (segment (start 97.536 118.11) (end 92.7497 113.3237) (width 0.2) (layer "F.Cu") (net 2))
 (segment (start 105.695074 108.204) (end 106.68 108.204) (width 0.2) (layer "F.Cu") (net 2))
 (segment (start 105.545374 103.124) (end 108.204 103.124) (width 0.2) (layer "F.Cu") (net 2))
 (segment (start 97.536 128.778) (end 97.38695 128.778) (width 0.2) (layer "F.Cu") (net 2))
 (segment (start 97.536 107.32235) (end 97.536 108.458) (width 0.2) (layer "F.Cu") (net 2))
 (segment (start 82.656 91.719) (end 81.105 93.27) (width 0.2) (layer "F.Cu") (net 2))
 (segment (start 82.656 102.52135) (end 81.105 104.07235) (width 0.2) (layer "F.Cu") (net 2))
 (segment (start 106.68 108.204) (end 108.204 106.68) (width 0.2) (layer "F.Cu") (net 2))
 (segment (start 97.536 128.778) (end 98.236 128.078) (width 0.2) (layer "F.Cu") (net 2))
 (segment (start 82.656 113.3237) (end 81.105 114.8747) (width 0.2) (layer "F.Cu") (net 2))
 (segment (start 98.8251 118.11) (end 101.6 115.3351) (width 0.2) (layer "F.Cu") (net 2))
 (segment (start 105.000972 110.744) (end 106.568763 110.744) (width 0.2) (layer "F.Cu") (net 2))
 (segment (start 104.648 104.021374) (end 105.545374 103.124) (width 0.2) (layer "F.Cu") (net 2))
 (segment (start 104.606177 107.908177) (end 104.606177 106.783968) (width 0.2) (layer "F.Cu") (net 2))
 (segment (start 97.5614 85.74705) (end 92.731 80.91665) (width 0.2) (layer "F.Cu") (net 2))
 (segment (start 97.5614 85.74705) (end 104.648 92.83365) (width 0.2) (layer "F.Cu") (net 2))
 (segment (start 103.41298 109.101374) (end 104.606177 107.908177) (width 0.2) (layer "F.Cu") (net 2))
 (segment (start 92.735 124.12605) (end 82.656 124.12605) (width 0.2) (layer "F.Cu") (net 2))
 (segment (start 102.474904 113.270068) (end 105.000972 110.744) (width 0.2) (layer "F.Cu") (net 2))
 (segment (start 131.51908 91.89508) (end 131.572 91.948) (width 0.2) (layer "F.Cu") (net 4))
 (segment (start 84.605 121.3747) (end 86.205 121.3747) (width 0.2) (layer "F.Cu") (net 4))
 (segment (start 90.954 130.28) (end 98.15815 130.28) (width 0.2) (layer "F.Cu") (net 4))
 (segment (start 147.805 90.401) (end 149.944 92.54) (width 0.2) (layer "F.Cu") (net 4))
 (segment (start 103.276904 113.602268) (end 103.773798 113.105374) (width 0.2) (layer "F.Cu") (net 4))
 (segment (start 243.84 112.118) (end 243.944 112.118) (width 0.2) (layer "F.Cu") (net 4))
 (segment (start 78.105 93.27) (end 84.605 99.77) (width 0.2) (layer "F.Cu") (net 4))
 (segment (start 84.605 99.77) (end 86.205 99.77) (width 0.2) (layer "F.Cu") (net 4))
 (segment (start 103.773798 113.105374) (end 107.112626 113.105374) (width 0.2) (layer "F.Cu") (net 4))
 (segment (start 98.15815 130.28) (end 99.038 129.40015) (width 0.2) (layer "F.Cu") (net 4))
 (segment (start 131.51908 91.722374) (end 131.51908 91.89508) (width 0.2) (layer "F.Cu") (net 4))
 (segment (start 240.642 115.316) (end 243.84 112.118) (width 0.2) (layer "F.Cu") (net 4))
 (segment (start 240.59 101.31) (end 243.84 104.56) (width 0.2) (layer "F.Cu") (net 4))
 (segment (start 243.944 112.118) (end 247.142 115.316) (width 0.2) (layer "F.Cu") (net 4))
 (segment (start 84.605 110.57235) (end 86.205 110.57235) (width 0.2) (layer "F.Cu") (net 4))
 (segment (start 78.105 82.46765) (end 84.605 88.96765) (width 0.2) (layer "F.Cu") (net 4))
 (segment (start 78.105 104.07235) (end 84.605 110.57235) (width 0.2) (layer "F.Cu") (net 4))
 (segment (start 134.391454 88.85) (end 139.812 88.85) (width 0.2) (layer "F.Cu") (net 4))
 (segment (start 139.812 88.85) (end 143.9089 88.85) (width 0.2) (layer "F.Cu") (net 4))
 (segment (start 99.038 120.1655) (end 103.276904 115.926596) (width 0.2) (layer "F.Cu") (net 4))
 (segment (start 78.105 114.8747) (end 84.605 121.3747) (width 0.2) (layer "F.Cu") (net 4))
 (segment (start 86.205 132.17705) (end 89.05695 132.17705) (width 0.2) (layer "F.Cu") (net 4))
 (segment (start 108.605 99.7341) (end 116.616726 91.722374) (width 0.2) (layer "F.Cu") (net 4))
 (segment (start 78.105 104.07235) (end 78.105 93.27) (width 0.2) (layer "F.Cu") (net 4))
 (segment (start 99.038 129.40015) (end 99.038 120.1655) (width 0.2) (layer "F.Cu") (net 4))
 (segment (start 247.09 101.31) (end 243.84 104.56) (width 0.2) (layer "F.Cu") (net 4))
 (segment (start 145.4599 90.401) (end 147.805 90.401) (width 0.2) (layer "F.Cu") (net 4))
 (segment (start 131.51908 91.722374) (end 134.391454 88.85) (width 0.2) (layer "F.Cu") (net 4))
 (segment (start 240.59 101.31) (end 231.82 92.54) (width 0.2) (layer "F.Cu") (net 4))
 (segment (start 143.9089 88.85) (end 145.4599 90.401) (width 0.2) (layer "F.Cu") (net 4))
 (segment (start 243.84 112.118) (end 243.84 111.506) (width 0.2) (layer "F.Cu") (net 4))
 (segment (start 89.05695 132.17705) (end 90.954 130.28) (width 0.2) (layer "F.Cu") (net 4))
 (segment (start 231.82 92.54) (end 151 92.54) (width 0.2) (layer "F.Cu") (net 4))
 (segment (start 243.84 111.506) (end 243.84 104.56) (width 0.2) (layer "F.Cu") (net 4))
 (segment (start 116.616726 91.722374) (end 131.51908 91.722374) (width 0.2) (layer "F.Cu") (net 4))
 (segment (start 78.105 114.8747) (end 78.105 104.07235) (width 0.2) (layer "F.Cu") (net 4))
 (segment (start 78.105 93.27) (end 78.105 82.46765) (width 0.2) (layer "F.Cu") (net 4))
 (segment (start 86.205 132.17705) (end 84.605 132.17705) (width 0.2) (layer "F.Cu") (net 4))
 (segment (start 108.605 111.613) (end 108.605 99.7341) (width 0.2) (layer "F.Cu") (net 4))
 (segment (start 84.605 88.96765) (end 86.205 88.96765) (width 0.2) (layer "F.Cu") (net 4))
 (segment (start 78.105 125.67705) (end 78.105 114.8747) (width 0.2) (layer "F.Cu") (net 4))
 (segment (start 84.605 132.17705) (end 78.105 125.67705) (width 0.2) (layer "F.Cu") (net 4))
 (segment (start 107.112626 113.105374) (end 108.605 111.613) (width 0.2) (layer "F.Cu") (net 4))
 (segment (start 149.944 92.54) (end 151 92.54) (width 0.2) (layer "F.Cu") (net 4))
 (segment (start 103.276904 115.926596) (end 103.276904 113.602268) (width 0.2) (layer "F.Cu") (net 4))
 (segment (start 130.048 96.012) (end 130.048 105.491294) (width 0.2) (layer "F.Cu") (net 6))
 (segment (start 130.048 105.491294) (end 131.51908 106.962374) (width 0.2) (layer "F.Cu") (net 6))
 (segment (start 130.556 95.504) (end 150.576 95.504) (width 0.2) (layer "F.Cu") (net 6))
 (segment (start 130.556 95.504) (end 130.048 96.012) (width 0.2) (layer "F.Cu") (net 6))
 (segment (start 150.576 95.504) (end 151 95.08) (width 0.2) (layer "F.Cu") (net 6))
 (segment (start 132.956727 111.171827) (end 132.986277 111.142277) (width 0.2) (layer "F.Cu") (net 9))
 (segment (start 132.986277 111.142277) (end 133.745554 110.383) (width 0.2) (layer "F.Cu") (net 9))
 (segment (start 130.81 113.284) (end 130.048 114.046) (width 0.2) (layer "F.Cu") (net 9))
 (segment (start 130.048 114.046) (end 130.048 123.952) (width 0.2) (layer "F.Cu") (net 9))
 (segment (start 132.08 113.284) (end 130.81 113.284) (width 0.2) (layer "F.Cu") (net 9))
 (segment (start 132.986277 112.377723) (end 132.08 113.284) (width 0.2) (layer "F.Cu") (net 9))
 (segment (start 130.048 123.952) (end 130.838374 124.742374) (width 0.2) (layer "F.Cu") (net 9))
 (segment (start 149.578 111.371) (end 152.185338 111.371) (width 0.2) (layer "F.Cu") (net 9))
 (segment (start 151 102.7) (end 153.162 104.862) (width 0.2) (layer "F.Cu") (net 9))
 (segment (start 130.838374 124.742374) (end 131.51908 124.742374) (width 0.2) (layer "F.Cu") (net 9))
 (segment (start 132.986277 111.142277) (end 132.986277 112.377723) (width 0.2) (layer "F.Cu") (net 9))
 (segment (start 152.185338 111.371) (end 153.162 110.394338) (width 0.2) (layer "F.Cu") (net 9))
 (segment (start 133.745554 110.383) (end 148.59 110.383) (width 0.2) (layer "F.Cu") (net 9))
 (segment (start 153.162 110.394338) (end 153.162 104.862) (width 0.2) (layer "F.Cu") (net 9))
 (segment (start 148.59 110.383) (end 149.578 111.371) (width 0.2) (layer "F.Cu") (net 9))
 (segment (start 146.765999 109.474) (end 150.999999 105.24) (width 0.2) (layer "F.Cu") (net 10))
 (segment (start 150.999999 105.24) (end 151 105.24) (width 0.2) (layer "F.Cu") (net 10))
 (segment (start 131.51908 109.502374) (end 131.547454 109.474) (width 0.2) (layer "F.Cu") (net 10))
 (segment (start 131.547454 109.474) (end 146.765999 109.474) (width 0.2) (layer "F.Cu") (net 10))
 (segment (start 134.083626 101.882374) (end 136.398 99.568) (width 0.2) (layer "F.Cu") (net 7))
 (segment (start 149.052 99.568) (end 151 97.62) (width 0.2) (layer "F.Cu") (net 7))
 (segment (start 136.398 99.568) (end 149.052 99.568) (width 0.2) (layer "F.Cu") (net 7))
 (segment (start 131.51908 101.882374) (end 131.51908 102.05508) (width 0.2) (layer "F.Cu") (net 7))
 (segment (start 131.51908 101.882374) (end 134.083626 101.882374) (width 0.2) (layer "F.Cu") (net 7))
 (segment (start 131.51908 102.05508) (end 131.572 102.108) (width 0.2) (layer "F.Cu") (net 7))
 (segment (start 131.51908 104.422374) (end 132.305626 104.422374) (width 0.2) (layer "F.Cu") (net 8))
 (segment (start 132.305626 104.422374) (end 136.568 100.16) (width 0.2) (layer "F.Cu") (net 8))
 (segment (start 136.568 100.16) (end 151 100.16) (width 0.2) (layer "F.Cu") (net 8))
 (segment (start 235.236 125.222) (end 134.538706 125.222) (width 0.2) (layer "F.Cu") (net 18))
 (segment (start 240.642 119.816) (end 247.142 119.816) (width 0.2) (layer "F.Cu") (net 18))
 (segment (start 240.642 119.816) (end 235.236 125.222) (width 0.2) (layer "F.Cu") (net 18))
 (segment (start 134.538706 125.222) (end 131.51908 122.202374) (width 0.2) (layer "F.Cu") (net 18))
 (segment (start 240.792 117.602) (end 239.014 119.38) (width 0.2) (layer "F.Cu") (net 35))
 (segment (start 247.904 117.602) (end 240.792 117.602) (width 0.2) (layer "F.Cu") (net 35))
 (segment (start 239.014 119.38) (end 239.014 120.8769) (width 0.2) (layer "F.Cu") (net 35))
 (segment (start 235.0699 124.821) (end 134.704806 124.821) (width 0.2) (layer "F.Cu") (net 35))
 (segment (start 247.09 96.81) (end 248.666 98.386) (width 0.2) (layer "F.Cu") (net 35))
 (segment (start 248.666 116.84) (end 247.904 117.602) (width 0.2) (layer "F.Cu") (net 35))
 (segment (start 248.666 98.386) (end 248.666 116.84) (width 0.2) (layer "F.Cu") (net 35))
 (segment (start 133.096 123.212194) (end 133.096 116.159294) (width 0.2) (layer "F.Cu") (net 35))
 (segment (start 240.59 96.81) (end 247.09 96.81) (width 0.2) (layer "F.Cu") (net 35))
 (segment (start 134.704806 124.821) (end 133.096 123.212194) (width 0.2) (layer "F.Cu") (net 35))
 (segment (start 239.014 120.8769) (end 235.0699 124.821) (width 0.2) (layer "F.Cu") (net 35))
 (segment (start 133.096 116.159294) (end 131.51908 114.582374) (width 0.2) (layer "F.Cu") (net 35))
 (segment (start 148.798 109.982) (end 133.579454 109.982) (width 0.2) (layer "F.Cu") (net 11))
 (segment (start 151 107.78) (end 148.798 109.982) (width 0.2) (layer "F.Cu") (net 11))
 (segment (start 133.579454 109.982) (end 131.51908 112.042374) (width 0.2) (layer "F.Cu") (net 11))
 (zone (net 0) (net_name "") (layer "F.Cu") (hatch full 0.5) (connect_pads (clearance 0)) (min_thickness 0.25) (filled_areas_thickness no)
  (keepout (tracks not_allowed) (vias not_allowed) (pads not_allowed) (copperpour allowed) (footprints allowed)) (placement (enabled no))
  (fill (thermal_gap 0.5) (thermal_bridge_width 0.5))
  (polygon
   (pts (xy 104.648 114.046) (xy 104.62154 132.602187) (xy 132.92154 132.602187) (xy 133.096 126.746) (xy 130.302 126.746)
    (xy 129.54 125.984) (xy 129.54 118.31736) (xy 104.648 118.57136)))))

